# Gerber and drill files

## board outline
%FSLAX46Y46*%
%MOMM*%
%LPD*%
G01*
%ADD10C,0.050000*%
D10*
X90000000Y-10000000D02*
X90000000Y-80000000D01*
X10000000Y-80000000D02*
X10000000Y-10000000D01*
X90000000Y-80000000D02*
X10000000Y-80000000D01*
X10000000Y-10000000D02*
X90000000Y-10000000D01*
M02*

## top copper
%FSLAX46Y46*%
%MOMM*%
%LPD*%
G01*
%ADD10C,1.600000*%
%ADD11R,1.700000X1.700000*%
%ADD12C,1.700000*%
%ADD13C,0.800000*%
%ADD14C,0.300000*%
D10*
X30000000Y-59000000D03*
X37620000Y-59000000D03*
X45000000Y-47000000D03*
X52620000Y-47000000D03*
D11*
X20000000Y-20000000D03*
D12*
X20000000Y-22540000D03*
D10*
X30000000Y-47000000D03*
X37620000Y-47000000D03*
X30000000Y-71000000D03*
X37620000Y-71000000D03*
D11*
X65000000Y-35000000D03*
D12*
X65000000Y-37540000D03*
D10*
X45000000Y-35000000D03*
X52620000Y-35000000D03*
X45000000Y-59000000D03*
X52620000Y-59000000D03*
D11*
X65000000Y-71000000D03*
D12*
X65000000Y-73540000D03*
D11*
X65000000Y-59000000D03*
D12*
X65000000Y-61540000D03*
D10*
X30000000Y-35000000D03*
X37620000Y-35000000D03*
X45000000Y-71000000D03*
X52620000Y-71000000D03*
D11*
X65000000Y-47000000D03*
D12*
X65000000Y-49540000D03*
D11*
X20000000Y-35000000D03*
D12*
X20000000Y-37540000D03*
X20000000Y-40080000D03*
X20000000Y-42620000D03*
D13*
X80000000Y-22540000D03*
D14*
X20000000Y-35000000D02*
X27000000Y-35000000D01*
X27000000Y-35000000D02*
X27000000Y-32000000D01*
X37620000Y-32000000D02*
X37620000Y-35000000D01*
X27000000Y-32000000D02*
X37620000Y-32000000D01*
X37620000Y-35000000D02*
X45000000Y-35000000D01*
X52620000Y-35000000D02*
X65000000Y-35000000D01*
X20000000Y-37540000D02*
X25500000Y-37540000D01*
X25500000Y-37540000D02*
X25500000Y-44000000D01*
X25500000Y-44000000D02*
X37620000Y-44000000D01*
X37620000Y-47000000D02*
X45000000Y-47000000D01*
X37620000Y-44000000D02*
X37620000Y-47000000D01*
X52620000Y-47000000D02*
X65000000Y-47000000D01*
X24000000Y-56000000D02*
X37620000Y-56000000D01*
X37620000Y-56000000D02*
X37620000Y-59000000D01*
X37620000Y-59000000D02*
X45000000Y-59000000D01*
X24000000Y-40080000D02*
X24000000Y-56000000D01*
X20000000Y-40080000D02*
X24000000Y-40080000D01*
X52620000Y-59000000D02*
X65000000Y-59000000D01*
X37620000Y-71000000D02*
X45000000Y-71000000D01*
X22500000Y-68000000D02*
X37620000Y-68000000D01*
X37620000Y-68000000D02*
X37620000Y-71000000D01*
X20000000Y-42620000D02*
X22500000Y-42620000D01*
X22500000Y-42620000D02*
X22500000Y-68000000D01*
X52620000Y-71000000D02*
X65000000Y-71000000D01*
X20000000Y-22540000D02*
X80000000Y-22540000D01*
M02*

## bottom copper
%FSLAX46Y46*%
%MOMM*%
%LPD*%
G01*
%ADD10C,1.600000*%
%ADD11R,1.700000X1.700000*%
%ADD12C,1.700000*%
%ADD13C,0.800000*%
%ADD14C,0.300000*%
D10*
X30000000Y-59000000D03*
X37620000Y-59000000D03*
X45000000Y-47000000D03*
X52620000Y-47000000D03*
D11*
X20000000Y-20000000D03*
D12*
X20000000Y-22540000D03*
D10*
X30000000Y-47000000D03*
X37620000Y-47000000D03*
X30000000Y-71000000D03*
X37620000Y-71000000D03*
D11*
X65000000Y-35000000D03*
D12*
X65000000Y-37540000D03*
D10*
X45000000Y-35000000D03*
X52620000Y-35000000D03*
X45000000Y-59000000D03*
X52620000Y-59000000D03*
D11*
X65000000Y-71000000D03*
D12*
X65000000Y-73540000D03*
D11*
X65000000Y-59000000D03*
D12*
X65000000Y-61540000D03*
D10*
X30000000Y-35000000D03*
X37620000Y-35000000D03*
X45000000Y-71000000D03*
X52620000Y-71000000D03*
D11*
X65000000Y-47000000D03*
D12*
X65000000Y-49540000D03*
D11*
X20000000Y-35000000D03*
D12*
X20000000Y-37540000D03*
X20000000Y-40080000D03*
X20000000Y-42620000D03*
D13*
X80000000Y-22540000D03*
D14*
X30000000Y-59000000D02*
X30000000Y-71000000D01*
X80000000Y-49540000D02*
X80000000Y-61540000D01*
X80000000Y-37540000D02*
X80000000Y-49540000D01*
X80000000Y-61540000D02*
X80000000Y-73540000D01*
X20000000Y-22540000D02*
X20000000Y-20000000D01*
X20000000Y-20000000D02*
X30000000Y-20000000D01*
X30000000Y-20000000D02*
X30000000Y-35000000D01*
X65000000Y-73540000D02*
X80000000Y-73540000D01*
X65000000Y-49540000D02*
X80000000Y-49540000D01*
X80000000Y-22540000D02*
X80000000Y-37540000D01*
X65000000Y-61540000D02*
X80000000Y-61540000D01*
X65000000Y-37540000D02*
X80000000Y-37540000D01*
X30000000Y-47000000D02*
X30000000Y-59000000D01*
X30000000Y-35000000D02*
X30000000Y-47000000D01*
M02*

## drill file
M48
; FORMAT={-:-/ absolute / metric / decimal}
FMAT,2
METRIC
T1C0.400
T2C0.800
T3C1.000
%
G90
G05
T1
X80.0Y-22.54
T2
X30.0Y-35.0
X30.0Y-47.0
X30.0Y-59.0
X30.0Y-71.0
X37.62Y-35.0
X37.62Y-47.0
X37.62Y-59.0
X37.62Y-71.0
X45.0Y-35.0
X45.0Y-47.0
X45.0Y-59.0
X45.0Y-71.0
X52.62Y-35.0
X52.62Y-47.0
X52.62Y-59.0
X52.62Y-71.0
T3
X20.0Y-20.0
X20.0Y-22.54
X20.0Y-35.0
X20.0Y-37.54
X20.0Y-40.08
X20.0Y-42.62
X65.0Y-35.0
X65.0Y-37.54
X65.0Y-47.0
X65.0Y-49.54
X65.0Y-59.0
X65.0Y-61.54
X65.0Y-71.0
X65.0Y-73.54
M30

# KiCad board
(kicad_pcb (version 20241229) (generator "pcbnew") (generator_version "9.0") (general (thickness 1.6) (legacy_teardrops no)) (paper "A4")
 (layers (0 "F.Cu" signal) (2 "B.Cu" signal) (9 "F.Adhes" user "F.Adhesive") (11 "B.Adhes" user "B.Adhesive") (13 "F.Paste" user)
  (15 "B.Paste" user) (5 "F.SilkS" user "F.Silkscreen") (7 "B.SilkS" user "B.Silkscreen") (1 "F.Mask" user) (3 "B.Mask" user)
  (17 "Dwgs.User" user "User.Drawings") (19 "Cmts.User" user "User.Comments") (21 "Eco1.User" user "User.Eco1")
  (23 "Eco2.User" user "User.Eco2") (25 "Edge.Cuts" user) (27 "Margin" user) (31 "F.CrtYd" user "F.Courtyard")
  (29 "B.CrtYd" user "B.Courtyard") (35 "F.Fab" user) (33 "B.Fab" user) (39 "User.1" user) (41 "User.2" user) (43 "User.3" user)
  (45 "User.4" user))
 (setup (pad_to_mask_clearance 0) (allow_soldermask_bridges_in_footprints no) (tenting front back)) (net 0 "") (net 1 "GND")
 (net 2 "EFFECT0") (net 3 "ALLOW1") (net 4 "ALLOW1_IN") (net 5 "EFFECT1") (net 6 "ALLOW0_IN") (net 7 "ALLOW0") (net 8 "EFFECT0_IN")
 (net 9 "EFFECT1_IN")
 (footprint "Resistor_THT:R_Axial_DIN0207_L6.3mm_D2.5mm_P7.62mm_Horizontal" (layer "F.Cu") (at 30 59)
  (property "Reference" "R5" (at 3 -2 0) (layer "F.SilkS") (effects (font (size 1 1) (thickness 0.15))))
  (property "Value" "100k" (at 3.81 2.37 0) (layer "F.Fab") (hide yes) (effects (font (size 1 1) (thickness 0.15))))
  (pad "1" thru_hole circle (at 0 0) (size 1.6 1.6) (drill 0.8) (layers "*.Cu" "*.Mask") (remove_unused_layers no) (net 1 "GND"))
  (pad "2" thru_hole circle (at 7.62 0) (size 1.6 1.6) (drill 0.8) (layers "*.Cu" "*.Mask") (remove_unused_layers no) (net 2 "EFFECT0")))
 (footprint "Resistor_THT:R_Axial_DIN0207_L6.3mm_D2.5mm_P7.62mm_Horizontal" (layer "F.Cu") (at 45 47)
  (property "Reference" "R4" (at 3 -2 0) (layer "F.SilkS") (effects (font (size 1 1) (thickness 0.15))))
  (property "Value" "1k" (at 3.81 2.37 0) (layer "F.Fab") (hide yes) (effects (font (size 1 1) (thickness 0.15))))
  (pad "1" thru_hole circle (at 0 0) (size 1.6 1.6) (drill 0.8) (layers "*.Cu" "*.Mask") (remove_unused_layers no) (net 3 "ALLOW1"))
  (pad "2" thru_hole circle (at 7.62 0) (size 1.6 1.6) (drill 0.8) (layers "*.Cu" "*.Mask") (remove_unused_layers no) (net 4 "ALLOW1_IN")))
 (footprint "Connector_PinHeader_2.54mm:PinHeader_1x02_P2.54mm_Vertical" (layer "F.Cu") (at 20 20)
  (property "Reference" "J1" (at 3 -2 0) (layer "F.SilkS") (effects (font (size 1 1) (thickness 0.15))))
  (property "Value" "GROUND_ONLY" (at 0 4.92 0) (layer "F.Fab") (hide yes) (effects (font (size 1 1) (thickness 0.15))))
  (pad "1" thru_hole rect (at 0 0) (size 1.7 1.7) (drill 1) (layers "*.Cu" "*.Mask") (remove_unused_layers no) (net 1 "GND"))
  (pad "2" thru_hole circle (at 0 2.54) (size 1.7 1.7) (drill 1) (layers "*.Cu" "*.Mask") (remove_unused_layers no) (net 1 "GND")))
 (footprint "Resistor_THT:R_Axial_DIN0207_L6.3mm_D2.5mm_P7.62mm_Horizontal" (layer "F.Cu") (at 30 47)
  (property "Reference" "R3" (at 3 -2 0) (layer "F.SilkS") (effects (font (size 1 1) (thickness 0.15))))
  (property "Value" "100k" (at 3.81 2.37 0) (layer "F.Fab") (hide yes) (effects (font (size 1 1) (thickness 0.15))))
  (pad "1" thru_hole circle (at 0 0) (size 1.6 1.6) (drill 0.8) (layers "*.Cu" "*.Mask") (remove_unused_layers no) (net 1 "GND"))
  (pad "2" thru_hole circle (at 7.62 0) (size 1.6 1.6) (drill 0.8) (layers "*.Cu" "*.Mask") (remove_unused_layers no) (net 3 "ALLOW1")))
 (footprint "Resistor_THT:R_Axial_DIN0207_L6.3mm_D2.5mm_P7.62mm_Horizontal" (layer "F.Cu") (at 30 71)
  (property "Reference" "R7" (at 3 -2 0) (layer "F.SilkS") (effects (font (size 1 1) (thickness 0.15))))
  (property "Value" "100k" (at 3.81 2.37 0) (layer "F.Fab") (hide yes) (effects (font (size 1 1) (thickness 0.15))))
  (pad "1" thru_hole circle (at 0 0) (size 1.6 1.6) (drill 0.8) (layers "*.Cu" "*.Mask") (remove_unused_layers no) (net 1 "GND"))
  (pad "2" thru_hole circle (at 7.62 0) (size 1.6 1.6) (drill 0.8) (layers "*.Cu" "*.Mask") (remove_unused_layers no) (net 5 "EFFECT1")))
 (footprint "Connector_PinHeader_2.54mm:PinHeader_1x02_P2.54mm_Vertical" (layer "F.Cu") (at 65 35)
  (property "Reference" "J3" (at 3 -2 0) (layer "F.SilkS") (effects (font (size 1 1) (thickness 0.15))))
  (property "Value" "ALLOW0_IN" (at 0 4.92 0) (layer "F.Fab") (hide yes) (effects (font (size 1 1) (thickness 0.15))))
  (pad "1" thru_hole rect (at 0 0) (size 1.7 1.7) (drill 1) (layers "*.Cu" "*.Mask") (remove_unused_layers no) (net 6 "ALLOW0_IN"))
  (pad "2" thru_hole circle (at 0 2.54) (size 1.7 1.7) (drill 1) (layers "*.Cu" "*.Mask") (remove_unused_layers no) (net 1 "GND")))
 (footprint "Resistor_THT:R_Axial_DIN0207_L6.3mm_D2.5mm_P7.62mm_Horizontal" (layer "F.Cu") (at 45 35)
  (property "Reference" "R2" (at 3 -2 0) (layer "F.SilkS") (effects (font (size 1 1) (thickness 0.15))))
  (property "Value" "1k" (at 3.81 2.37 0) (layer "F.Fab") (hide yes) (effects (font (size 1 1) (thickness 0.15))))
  (pad "1" thru_hole circle (at 0 0) (size 1.6 1.6) (drill 0.8) (layers "*.Cu" "*.Mask") (remove_unused_layers no) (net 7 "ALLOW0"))
  (pad "2" thru_hole circle (at 7.62 0) (size 1.6 1.6) (drill 0.8) (layers "*.Cu" "*.Mask") (remove_unused_layers no) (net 6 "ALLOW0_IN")))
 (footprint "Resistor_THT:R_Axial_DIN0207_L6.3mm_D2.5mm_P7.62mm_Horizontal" (layer "F.Cu") (at 45 59)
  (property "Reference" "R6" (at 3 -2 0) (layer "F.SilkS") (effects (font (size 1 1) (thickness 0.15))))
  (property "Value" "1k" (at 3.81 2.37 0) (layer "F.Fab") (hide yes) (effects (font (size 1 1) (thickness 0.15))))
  (pad "1" thru_hole circle (at 0 0) (size 1.6 1.6) (drill 0.8) (layers "*.Cu" "*.Mask") (remove_unused_layers no) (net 2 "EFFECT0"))
  (pad "2" thru_hole circle (at 7.62 0) (size 1.6 1.6) (drill 0.8) (layers "*.Cu" "*.Mask") (remove_unused_layers no) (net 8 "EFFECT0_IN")))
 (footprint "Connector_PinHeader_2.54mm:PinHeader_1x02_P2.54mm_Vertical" (layer "F.Cu") (at 65 71)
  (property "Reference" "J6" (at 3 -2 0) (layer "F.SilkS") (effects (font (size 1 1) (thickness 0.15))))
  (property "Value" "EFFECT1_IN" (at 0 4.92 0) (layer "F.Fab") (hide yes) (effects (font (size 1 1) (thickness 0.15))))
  (pad "1" thru_hole rect (at 0 0) (size 1.7 1.7) (drill 1) (layers "*.Cu" "*.Mask") (remove_unused_layers no) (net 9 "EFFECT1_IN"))
  (pad "2" thru_hole circle (at 0 2.54) (size 1.7 1.7) (drill 1) (layers "*.Cu" "*.Mask") (remove_unused_layers no) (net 1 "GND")))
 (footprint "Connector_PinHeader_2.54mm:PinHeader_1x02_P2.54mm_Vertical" (layer "F.Cu") (at 65 59)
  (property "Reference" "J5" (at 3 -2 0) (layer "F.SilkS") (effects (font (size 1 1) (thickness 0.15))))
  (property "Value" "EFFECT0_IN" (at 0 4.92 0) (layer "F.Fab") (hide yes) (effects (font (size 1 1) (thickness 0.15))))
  (pad "1" thru_hole rect (at 0 0) (size 1.7 1.7) (drill 1) (layers "*.Cu" "*.Mask") (remove_unused_layers no) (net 8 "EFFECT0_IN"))
  (pad "2" thru_hole circle (at 0 2.54) (size 1.7 1.7) (drill 1) (layers "*.Cu" "*.Mask") (remove_unused_layers no) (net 1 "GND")))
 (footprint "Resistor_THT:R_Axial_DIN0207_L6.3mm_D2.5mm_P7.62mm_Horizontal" (layer "F.Cu") (at 30 35)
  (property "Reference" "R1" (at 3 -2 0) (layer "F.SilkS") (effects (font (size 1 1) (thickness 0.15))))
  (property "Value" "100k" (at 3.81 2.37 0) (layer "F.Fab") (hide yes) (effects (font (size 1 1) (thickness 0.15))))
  (pad "1" thru_hole circle (at 0 0) (size 1.6 1.6) (drill 0.8) (layers "*.Cu" "*.Mask") (remove_unused_layers no) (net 1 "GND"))
  (pad "2" thru_hole circle (at 7.62 0) (size 1.6 1.6) (drill 0.8) (layers "*.Cu" "*.Mask") (remove_unused_layers no) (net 7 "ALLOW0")))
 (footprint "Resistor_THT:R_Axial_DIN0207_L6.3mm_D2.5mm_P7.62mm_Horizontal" (layer "F.Cu") (at 45 71)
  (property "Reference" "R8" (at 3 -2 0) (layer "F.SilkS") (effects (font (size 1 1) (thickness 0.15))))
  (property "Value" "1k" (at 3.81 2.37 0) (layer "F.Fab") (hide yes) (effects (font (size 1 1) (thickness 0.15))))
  (pad "1" thru_hole circle (at 0 0) (size 1.6 1.6) (drill 0.8) (layers "*.Cu" "*.Mask") (remove_unused_layers no) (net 5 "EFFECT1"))
  (pad "2" thru_hole circle (at 7.62 0) (size 1.6 1.6) (drill 0.8) (layers "*.Cu" "*.Mask") (remove_unused_layers no) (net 9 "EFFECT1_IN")))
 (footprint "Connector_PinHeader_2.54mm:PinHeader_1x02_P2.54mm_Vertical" (layer "F.Cu") (at 65 47)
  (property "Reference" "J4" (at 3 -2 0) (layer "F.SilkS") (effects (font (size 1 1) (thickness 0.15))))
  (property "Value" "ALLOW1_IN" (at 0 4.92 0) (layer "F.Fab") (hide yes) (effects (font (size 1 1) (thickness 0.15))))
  (pad "1" thru_hole rect (at 0 0) (size 1.7 1.7) (drill 1) (layers "*.Cu" "*.Mask") (remove_unused_layers no) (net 4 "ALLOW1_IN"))
  (pad "2" thru_hole circle (at 0 2.54) (size 1.7 1.7) (drill 1) (layers "*.Cu" "*.Mask") (remove_unused_layers no) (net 1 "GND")))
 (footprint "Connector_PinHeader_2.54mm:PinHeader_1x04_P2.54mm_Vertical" (layer "F.Cu") (at 20 35)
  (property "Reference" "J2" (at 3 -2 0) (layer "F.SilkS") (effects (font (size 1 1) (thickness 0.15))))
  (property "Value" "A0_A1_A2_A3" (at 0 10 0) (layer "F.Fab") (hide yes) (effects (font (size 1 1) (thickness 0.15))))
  (pad "1" thru_hole rect (at 0 0) (size 1.7 1.7) (drill 1) (layers "*.Cu" "*.Mask") (remove_unused_layers no) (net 7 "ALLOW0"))
  (pad "2" thru_hole circle (at 0 2.54) (size 1.7 1.7) (drill 1) (layers "*.Cu" "*.Mask") (remove_unused_layers no) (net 3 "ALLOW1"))
  (pad "3" thru_hole circle (at 0 5.08) (size 1.7 1.7) (drill 1) (layers "*.Cu" "*.Mask") (remove_unused_layers no) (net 2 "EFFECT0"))
  (pad "4" thru_hole circle (at 0 7.62) (size 1.7 1.7) (drill 1) (layers "*.Cu" "*.Mask") (remove_unused_layers no) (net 5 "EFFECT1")))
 (gr_line (start 90 10) (end 90 80) (stroke (width 0.05) (type default)) (layer "Edge.Cuts"))
 (gr_line (start 10 80) (end 10 10) (stroke (width 0.05) (type default)) (layer "Edge.Cuts"))
 (gr_line (start 90 80) (end 10 80) (stroke (width 0.05) (type default)) (layer "Edge.Cuts"))
 (gr_line (start 10 10) (end 90 10) (stroke (width 0.05) (type default)) (layer "Edge.Cuts"))
 (segment (start 20 35) (end 27 35) (width 0.3) (layer "F.Cu") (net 7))
 (segment (start 27 35) (end 27 32) (width 0.3) (layer "F.Cu") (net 7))
 (segment (start 37.62 32) (end 37.62 35) (width 0.3) (layer "F.Cu") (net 7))
 (segment (start 27 32) (end 37.62 32) (width 0.3) (layer "F.Cu") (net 7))
 (segment (start 37.62 35) (end 45 35) (width 0.3) (layer "F.Cu") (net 7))
 (segment (start 52.62 35) (end 65 35) (width 0.3) (layer "F.Cu") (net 6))
 (segment (start 20 37.54) (end 25.5 37.54) (width 0.3) (layer "F.Cu") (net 3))
 (segment (start 25.5 37.54) (end 25.5 44) (width 0.3) (layer "F.Cu") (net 3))
 (segment (start 25.5 44) (end 37.62 44) (width 0.3) (layer "F.Cu") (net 3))
 (segment (start 37.62 47) (end 45 47) (width 0.3) (layer "F.Cu") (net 3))
 (segment (start 37.62 44) (end 37.62 47) (width 0.3) (layer "F.Cu") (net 3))
 (segment (start 52.62 47) (end 65 47) (width 0.3) (layer "F.Cu") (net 4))
 (segment (start 24 56) (end 37.62 56) (width 0.3) (layer "F.Cu") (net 2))
 (segment (start 37.62 56) (end 37.62 59) (width 0.3) (layer "F.Cu") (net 2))
 (segment (start 37.62 59) (end 45 59) (width 0.3) (layer "F.Cu") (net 2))
 (segment (start 24 40.08) (end 24 56) (width 0.3) (layer "F.Cu") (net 2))
 (segment (start 20 40.08) (end 24 40.08) (width 0.3) (layer "F.Cu") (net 2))
 (segment (start 52.62 59) (end 65 59) (width 0.3) (layer "F.Cu") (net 8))
 (segment (start 37.62 71) (end 45 71) (width 0.3) (layer "F.Cu") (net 5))
 (segment (start 22.5 68) (end 37.62 68) (width 0.3) (layer "F.Cu") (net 5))
 (segment (start 37.62 68) (end 37.62 71) (width 0.3) (layer "F.Cu") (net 5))
 (segment (start 20 42.62) (end 22.5 42.62) (width 0.3) (layer "F.Cu") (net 5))
 (segment (start 22.5 42.62) (end 22.5 68) (width 0.3) (layer "F.Cu") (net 5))
 (segment (start 52.62 71) (end 65 71) (width 0.3) (layer "F.Cu") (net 9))
 (segment (start 20 22.54) (end 80 22.54) (width 0.3) (layer "F.Cu") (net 1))
 (via (at 80 22.54) (size 0.8) (drill 0.4) (layers "F.Cu" "B.Cu") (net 1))
 (segment (start 30 59) (end 30 71) (width 0.3) (layer "B.Cu") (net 1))
 (segment (start 80 49.54) (end 80 61.54) (width 0.3) (layer "B.Cu") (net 1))
 (segment (start 80 37.54) (end 80 49.54) (width 0.3) (layer "B.Cu") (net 1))
 (segment (start 80 61.54) (end 80 73.54) (width 0.3) (layer "B.Cu") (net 1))
 (segment (start 20 22.54) (end 20 20) (width 0.3) (layer "B.Cu") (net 1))
 (segment (start 20 20) (end 30 20) (width 0.3) (layer "B.Cu") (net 1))
 (segment (start 30 20) (end 30 35) (width 0.3) (layer "B.Cu") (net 1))
 (segment (start 65 73.54) (end 80 73.54) (width 0.3) (layer "B.Cu") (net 1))
 (segment (start 65 49.54) (end 80 49.54) (width 0.3) (layer "B.Cu") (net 1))
 (segment (start 80 22.54) (end 80 37.54) (width 0.3) (layer "B.Cu") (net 1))
 (segment (start 65 61.54) (end 80 61.54) (width 0.3) (layer "B.Cu") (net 1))
 (segment (start 65 37.54) (end 80 37.54) (width 0.3) (layer "B.Cu") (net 1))
 (segment (start 30 47) (end 30 59) (width 0.3) (layer "B.Cu") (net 1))
 (segment (start 30 35) (end 30 47) (width 0.3) (layer "B.Cu") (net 1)))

